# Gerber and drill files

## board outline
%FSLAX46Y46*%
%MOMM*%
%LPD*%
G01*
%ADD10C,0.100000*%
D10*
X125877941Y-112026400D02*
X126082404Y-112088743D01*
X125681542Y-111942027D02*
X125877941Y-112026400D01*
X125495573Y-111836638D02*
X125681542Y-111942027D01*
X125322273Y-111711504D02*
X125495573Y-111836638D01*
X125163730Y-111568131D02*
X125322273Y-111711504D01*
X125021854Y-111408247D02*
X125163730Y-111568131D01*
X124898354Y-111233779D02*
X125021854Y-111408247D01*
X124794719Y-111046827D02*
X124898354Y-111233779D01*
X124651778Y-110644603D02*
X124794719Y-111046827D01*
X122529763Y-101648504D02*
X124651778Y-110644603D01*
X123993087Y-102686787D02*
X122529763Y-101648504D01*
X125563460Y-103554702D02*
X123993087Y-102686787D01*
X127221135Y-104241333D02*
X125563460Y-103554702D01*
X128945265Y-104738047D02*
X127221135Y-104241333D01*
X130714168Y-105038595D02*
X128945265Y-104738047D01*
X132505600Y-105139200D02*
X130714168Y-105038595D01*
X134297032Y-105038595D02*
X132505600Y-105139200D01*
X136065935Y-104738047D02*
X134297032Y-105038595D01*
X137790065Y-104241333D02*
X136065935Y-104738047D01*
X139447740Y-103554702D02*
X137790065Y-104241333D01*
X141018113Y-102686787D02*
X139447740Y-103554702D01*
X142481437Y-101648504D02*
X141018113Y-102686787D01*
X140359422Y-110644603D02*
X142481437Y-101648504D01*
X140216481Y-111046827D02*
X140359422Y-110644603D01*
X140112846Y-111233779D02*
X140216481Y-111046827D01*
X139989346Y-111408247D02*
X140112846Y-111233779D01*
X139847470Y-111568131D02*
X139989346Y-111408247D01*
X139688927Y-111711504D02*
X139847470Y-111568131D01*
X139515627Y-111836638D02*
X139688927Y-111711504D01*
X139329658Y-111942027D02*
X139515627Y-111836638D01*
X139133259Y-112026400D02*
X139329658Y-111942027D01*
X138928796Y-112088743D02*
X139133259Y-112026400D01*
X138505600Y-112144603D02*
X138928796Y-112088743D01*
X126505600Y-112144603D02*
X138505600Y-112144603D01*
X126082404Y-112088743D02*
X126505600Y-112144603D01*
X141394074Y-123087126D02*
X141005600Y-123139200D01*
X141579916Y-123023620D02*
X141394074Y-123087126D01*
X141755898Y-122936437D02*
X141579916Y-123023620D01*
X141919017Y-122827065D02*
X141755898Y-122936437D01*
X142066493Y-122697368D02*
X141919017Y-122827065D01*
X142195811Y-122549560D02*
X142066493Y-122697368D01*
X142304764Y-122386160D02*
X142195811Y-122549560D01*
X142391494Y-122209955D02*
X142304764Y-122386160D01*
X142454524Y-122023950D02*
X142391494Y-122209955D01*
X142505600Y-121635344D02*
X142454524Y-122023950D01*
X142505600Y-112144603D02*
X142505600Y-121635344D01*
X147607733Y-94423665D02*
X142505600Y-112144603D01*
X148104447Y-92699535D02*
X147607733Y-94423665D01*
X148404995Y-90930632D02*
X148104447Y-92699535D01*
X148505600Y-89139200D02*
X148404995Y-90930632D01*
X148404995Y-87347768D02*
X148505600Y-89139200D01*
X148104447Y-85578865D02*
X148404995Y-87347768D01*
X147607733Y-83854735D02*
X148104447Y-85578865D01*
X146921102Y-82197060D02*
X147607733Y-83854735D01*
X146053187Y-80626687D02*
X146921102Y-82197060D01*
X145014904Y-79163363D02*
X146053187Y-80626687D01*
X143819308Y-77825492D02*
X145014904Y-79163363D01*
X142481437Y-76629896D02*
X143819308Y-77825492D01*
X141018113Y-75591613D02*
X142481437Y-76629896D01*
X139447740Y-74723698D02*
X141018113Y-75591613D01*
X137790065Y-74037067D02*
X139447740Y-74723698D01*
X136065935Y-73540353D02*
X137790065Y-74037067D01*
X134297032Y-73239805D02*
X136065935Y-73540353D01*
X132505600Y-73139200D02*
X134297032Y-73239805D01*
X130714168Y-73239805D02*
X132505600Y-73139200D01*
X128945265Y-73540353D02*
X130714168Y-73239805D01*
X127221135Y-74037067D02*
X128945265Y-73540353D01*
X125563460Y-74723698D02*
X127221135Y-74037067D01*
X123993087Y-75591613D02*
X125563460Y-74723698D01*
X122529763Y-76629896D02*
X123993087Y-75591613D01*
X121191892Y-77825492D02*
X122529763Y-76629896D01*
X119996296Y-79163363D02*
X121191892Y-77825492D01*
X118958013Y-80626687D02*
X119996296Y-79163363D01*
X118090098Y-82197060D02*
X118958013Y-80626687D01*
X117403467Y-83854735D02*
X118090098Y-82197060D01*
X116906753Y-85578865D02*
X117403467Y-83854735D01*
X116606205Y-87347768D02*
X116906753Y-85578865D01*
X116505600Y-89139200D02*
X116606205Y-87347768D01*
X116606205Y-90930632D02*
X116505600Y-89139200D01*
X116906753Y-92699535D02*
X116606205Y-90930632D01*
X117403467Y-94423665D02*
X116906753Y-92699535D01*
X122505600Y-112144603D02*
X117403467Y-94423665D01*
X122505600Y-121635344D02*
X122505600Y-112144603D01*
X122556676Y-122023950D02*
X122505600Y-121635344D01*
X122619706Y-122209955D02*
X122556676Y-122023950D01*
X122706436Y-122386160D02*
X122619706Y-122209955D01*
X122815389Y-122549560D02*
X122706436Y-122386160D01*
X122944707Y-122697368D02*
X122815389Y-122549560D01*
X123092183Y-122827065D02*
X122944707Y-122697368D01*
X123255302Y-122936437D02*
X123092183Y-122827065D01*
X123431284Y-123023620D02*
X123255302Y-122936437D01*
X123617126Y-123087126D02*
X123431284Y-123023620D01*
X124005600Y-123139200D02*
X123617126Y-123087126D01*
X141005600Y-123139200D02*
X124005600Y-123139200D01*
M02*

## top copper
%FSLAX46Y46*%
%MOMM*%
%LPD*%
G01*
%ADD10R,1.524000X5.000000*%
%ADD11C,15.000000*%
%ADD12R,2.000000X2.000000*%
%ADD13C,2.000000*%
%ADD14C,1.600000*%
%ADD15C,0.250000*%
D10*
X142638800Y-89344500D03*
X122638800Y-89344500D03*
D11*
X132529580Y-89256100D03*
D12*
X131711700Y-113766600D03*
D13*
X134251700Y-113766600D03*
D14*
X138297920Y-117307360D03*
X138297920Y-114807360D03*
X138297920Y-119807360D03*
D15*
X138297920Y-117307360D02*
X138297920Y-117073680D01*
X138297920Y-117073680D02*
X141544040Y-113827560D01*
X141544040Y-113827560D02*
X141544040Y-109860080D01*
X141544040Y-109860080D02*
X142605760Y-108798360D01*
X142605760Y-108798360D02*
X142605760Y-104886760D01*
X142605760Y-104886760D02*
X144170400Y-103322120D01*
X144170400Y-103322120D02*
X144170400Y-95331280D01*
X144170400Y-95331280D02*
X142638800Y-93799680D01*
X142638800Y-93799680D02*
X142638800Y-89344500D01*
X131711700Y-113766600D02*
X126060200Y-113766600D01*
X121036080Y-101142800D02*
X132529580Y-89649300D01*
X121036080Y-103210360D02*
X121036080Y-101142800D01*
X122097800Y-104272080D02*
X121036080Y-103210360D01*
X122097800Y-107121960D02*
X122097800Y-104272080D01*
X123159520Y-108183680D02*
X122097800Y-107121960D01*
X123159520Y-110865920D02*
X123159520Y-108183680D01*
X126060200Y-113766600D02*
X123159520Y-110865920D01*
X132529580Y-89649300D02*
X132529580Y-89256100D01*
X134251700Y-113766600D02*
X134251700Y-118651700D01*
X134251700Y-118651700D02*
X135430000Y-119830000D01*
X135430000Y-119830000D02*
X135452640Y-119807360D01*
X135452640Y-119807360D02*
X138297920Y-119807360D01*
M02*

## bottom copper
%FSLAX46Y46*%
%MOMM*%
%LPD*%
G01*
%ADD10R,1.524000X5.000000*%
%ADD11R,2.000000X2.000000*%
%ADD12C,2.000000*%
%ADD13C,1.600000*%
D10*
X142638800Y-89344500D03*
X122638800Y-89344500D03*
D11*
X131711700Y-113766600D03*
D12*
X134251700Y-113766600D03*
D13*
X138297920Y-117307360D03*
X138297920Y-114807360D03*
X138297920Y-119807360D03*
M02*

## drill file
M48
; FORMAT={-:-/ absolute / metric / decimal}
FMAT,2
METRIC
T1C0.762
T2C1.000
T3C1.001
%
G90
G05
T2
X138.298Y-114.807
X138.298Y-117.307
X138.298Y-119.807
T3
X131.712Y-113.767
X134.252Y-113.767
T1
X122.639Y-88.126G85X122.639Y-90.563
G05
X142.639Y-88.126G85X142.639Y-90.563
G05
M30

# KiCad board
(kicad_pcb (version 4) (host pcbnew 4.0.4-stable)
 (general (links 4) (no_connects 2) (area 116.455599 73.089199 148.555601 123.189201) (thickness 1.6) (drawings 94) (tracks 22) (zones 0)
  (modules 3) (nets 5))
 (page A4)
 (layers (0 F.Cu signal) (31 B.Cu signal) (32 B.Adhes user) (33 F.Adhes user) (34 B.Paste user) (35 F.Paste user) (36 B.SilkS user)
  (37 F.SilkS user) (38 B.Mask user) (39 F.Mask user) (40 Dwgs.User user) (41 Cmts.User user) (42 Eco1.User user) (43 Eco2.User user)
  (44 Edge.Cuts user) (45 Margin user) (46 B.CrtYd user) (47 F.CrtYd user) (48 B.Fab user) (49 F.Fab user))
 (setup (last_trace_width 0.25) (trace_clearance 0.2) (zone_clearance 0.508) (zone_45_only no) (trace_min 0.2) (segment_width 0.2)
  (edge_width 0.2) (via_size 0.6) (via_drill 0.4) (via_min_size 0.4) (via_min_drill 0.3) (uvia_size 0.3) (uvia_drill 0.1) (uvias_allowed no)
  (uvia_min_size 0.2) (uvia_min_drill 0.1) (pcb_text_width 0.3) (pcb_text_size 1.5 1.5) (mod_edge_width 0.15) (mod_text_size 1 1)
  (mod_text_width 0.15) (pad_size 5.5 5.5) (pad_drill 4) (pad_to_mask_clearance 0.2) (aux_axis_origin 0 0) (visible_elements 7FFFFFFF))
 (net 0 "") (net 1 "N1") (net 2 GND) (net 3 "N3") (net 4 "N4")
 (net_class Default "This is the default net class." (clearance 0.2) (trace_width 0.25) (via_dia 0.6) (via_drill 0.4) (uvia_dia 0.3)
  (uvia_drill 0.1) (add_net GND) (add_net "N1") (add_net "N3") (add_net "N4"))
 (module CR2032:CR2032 (layer F.Cu) (at 132.6388 89.3445)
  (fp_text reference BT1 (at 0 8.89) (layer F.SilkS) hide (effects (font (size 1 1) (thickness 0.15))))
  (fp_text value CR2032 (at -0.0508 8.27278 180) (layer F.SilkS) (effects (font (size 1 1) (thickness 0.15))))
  (pad 1 thru_hole rect (at 10 0) (size 1.524 5) (drill oval 0.762 3.2) (layers *.Cu *.Mask F.SilkS) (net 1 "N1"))
  (pad 1 thru_hole rect (at -10 0) (size 1.524 5) (drill oval 0.762 3.2) (layers *.Cu *.Mask F.SilkS) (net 1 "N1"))
  (pad 2 smd circle (at -0.10922 -0.0884) (size 15 15) (layers F.Cu F.Paste F.Mask) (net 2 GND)))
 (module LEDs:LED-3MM (layer F.Cu) (at 131.7117 113.7666)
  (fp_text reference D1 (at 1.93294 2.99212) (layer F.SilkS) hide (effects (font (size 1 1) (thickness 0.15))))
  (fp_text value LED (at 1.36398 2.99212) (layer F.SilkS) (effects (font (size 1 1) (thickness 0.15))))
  (pad 1 thru_hole rect (at 0 0 90) (size 2 2) (drill 1.00076) (layers *.Cu *.Mask F.SilkS) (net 2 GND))
  (pad 2 thru_hole circle (at 2.54 0) (size 2 2) (drill 1.00076) (layers *.Cu *.Mask F.SilkS) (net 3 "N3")))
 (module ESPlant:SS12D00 (layer F.Cu) (at 138.29792 117.30736 270)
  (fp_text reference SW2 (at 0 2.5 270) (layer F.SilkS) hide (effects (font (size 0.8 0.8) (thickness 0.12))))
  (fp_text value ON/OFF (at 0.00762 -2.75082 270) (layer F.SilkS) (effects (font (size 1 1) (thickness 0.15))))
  (pad 2 thru_hole circle (at 0 0 270) (size 1.6 1.6) (drill 1) (layers *.Cu *.Mask F.SilkS) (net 1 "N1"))
  (pad 1 thru_hole circle (at -2.5 0 270) (size 1.6 1.6) (drill 1) (layers *.Cu *.Mask F.SilkS) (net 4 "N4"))
  (pad 3 thru_hole circle (at 2.5 0 270) (size 1.6 1.6) (drill 1) (layers *.Cu *.Mask F.SilkS) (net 3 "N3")))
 (gr_line (start 125.877941 112.0264) (end 126.082404 112.088743) (layer Edge.Cuts) (width 0.1))
 (gr_line (start 125.681542 111.942027) (end 125.877941 112.0264) (layer Edge.Cuts) (width 0.1))
 (gr_line (start 125.495573 111.836638) (end 125.681542 111.942027) (layer Edge.Cuts) (width 0.1))
 (gr_line (start 125.322273 111.711504) (end 125.495573 111.836638) (layer Edge.Cuts) (width 0.1))
 (gr_line (start 125.16373 111.568131) (end 125.322273 111.711504) (layer Edge.Cuts) (width 0.1))
 (gr_line (start 125.021854 111.408247) (end 125.16373 111.568131) (layer Edge.Cuts) (width 0.1))
 (gr_line (start 124.898354 111.233779) (end 125.021854 111.408247) (layer Edge.Cuts) (width 0.1))
 (gr_line (start 124.794719 111.046827) (end 124.898354 111.233779) (layer Edge.Cuts) (width 0.1))
 (gr_line (start 124.651778 110.644603) (end 124.794719 111.046827) (layer Edge.Cuts) (width 0.1))
 (gr_line (start 122.529763 101.648504) (end 124.651778 110.644603) (layer Edge.Cuts) (width 0.1))
 (gr_line (start 123.993087 102.686787) (end 122.529763 101.648504) (layer Edge.Cuts) (width 0.1))
 (gr_line (start 125.56346 103.554702) (end 123.993087 102.686787) (layer Edge.Cuts) (width 0.1))
 (gr_line (start 127.221135 104.241333) (end 125.56346 103.554702) (layer Edge.Cuts) (width 0.1))
 (gr_line (start 128.945265 104.738047) (end 127.221135 104.241333) (layer Edge.Cuts) (width 0.1))
 (gr_line (start 130.714168 105.038595) (end 128.945265 104.738047) (layer Edge.Cuts) (width 0.1))
 (gr_line (start 132.5056 105.1392) (end 130.714168 105.038595) (layer Edge.Cuts) (width 0.1))
 (gr_line (start 134.297032 105.038595) (end 132.5056 105.1392) (layer Edge.Cuts) (width 0.1))
 (gr_line (start 136.065935 104.738047) (end 134.297032 105.038595) (layer Edge.Cuts) (width 0.1))
 (gr_line (start 137.790065 104.241333) (end 136.065935 104.738047) (layer Edge.Cuts) (width 0.1))
 (gr_line (start 139.44774 103.554702) (end 137.790065 104.241333) (layer Edge.Cuts) (width 0.1))
 (gr_line (start 141.018113 102.686787) (end 139.44774 103.554702) (layer Edge.Cuts) (width 0.1))
 (gr_line (start 142.481437 101.648504) (end 141.018113 102.686787) (layer Edge.Cuts) (width 0.1))
 (gr_line (start 140.359422 110.644603) (end 142.481437 101.648504) (layer Edge.Cuts) (width 0.1))
 (gr_line (start 140.216481 111.046827) (end 140.359422 110.644603) (layer Edge.Cuts) (width 0.1))
 (gr_line (start 140.112846 111.233779) (end 140.216481 111.046827) (layer Edge.Cuts) (width 0.1))
 (gr_line (start 139.989346 111.408247) (end 140.112846 111.233779) (layer Edge.Cuts) (width 0.1))
 (gr_line (start 139.84747 111.568131) (end 139.989346 111.408247) (layer Edge.Cuts) (width 0.1))
 (gr_line (start 139.688927 111.711504) (end 139.84747 111.568131) (layer Edge.Cuts) (width 0.1))
 (gr_line (start 139.515627 111.836638) (end 139.688927 111.711504) (layer Edge.Cuts) (width 0.1))
 (gr_line (start 139.329658 111.942027) (end 139.515627 111.836638) (layer Edge.Cuts) (width 0.1))
 (gr_line (start 139.133259 112.0264) (end 139.329658 111.942027) (layer Edge.Cuts) (width 0.1))
 (gr_line (start 138.928796 112.088743) (end 139.133259 112.0264) (layer Edge.Cuts) (width 0.1))
 (gr_line (start 138.5056 112.144603) (end 138.928796 112.088743) (layer Edge.Cuts) (width 0.1))
 (gr_line (start 126.5056 112.144603) (end 138.5056 112.144603) (layer Edge.Cuts) (width 0.1))
 (gr_line (start 126.082404 112.088743) (end 126.5056 112.144603) (layer Edge.Cuts) (width 0.1))
 (gr_line (start 141.394074 123.087126) (end 141.0056 123.1392) (layer Edge.Cuts) (width 0.1))
 (gr_line (start 141.579916 123.02362) (end 141.394074 123.087126) (layer Edge.Cuts) (width 0.1))
 (gr_line (start 141.755898 122.936437) (end 141.579916 123.02362) (layer Edge.Cuts) (width 0.1))
 (gr_line (start 141.919017 122.827065) (end 141.755898 122.936437) (layer Edge.Cuts) (width 0.1))
 (gr_line (start 142.066493 122.697368) (end 141.919017 122.827065) (layer Edge.Cuts) (width 0.1))
 (gr_line (start 142.195811 122.54956) (end 142.066493 122.697368) (layer Edge.Cuts) (width 0.1))
 (gr_line (start 142.304764 122.38616) (end 142.195811 122.54956) (layer Edge.Cuts) (width 0.1))
 (gr_line (start 142.391494 122.209955) (end 142.304764 122.38616) (layer Edge.Cuts) (width 0.1))
 (gr_line (start 142.454524 122.02395) (end 142.391494 122.209955) (layer Edge.Cuts) (width 0.1))
 (gr_line (start 142.5056 121.635344) (end 142.454524 122.02395) (layer Edge.Cuts) (width 0.1))
 (gr_line (start 142.5056 112.144603) (end 142.5056 121.635344) (layer Edge.Cuts) (width 0.1))
 (gr_line (start 147.607733 94.423665) (end 142.5056 112.144603) (layer Edge.Cuts) (width 0.1))
 (gr_line (start 148.104447 92.699535) (end 147.607733 94.423665) (layer Edge.Cuts) (width 0.1))
 (gr_line (start 148.404995 90.930632) (end 148.104447 92.699535) (layer Edge.Cuts) (width 0.1))
 (gr_line (start 148.5056 89.1392) (end 148.404995 90.930632) (layer Edge.Cuts) (width 0.1))
 (gr_line (start 148.404995 87.347768) (end 148.5056 89.1392) (layer Edge.Cuts) (width 0.1))
 (gr_line (start 148.104447 85.578865) (end 148.404995 87.347768) (layer Edge.Cuts) (width 0.1))
 (gr_line (start 147.607733 83.854735) (end 148.104447 85.578865) (layer Edge.Cuts) (width 0.1))
 (gr_line (start 146.921102 82.19706) (end 147.607733 83.854735) (layer Edge.Cuts) (width 0.1))
 (gr_line (start 146.053187 80.626687) (end 146.921102 82.19706) (layer Edge.Cuts) (width 0.1))
 (gr_line (start 145.014904 79.163363) (end 146.053187 80.626687) (layer Edge.Cuts) (width 0.1))
 (gr_line (start 143.819308 77.825492) (end 145.014904 79.163363) (layer Edge.Cuts) (width 0.1))
 (gr_line (start 142.481437 76.629896) (end 143.819308 77.825492) (layer Edge.Cuts) (width 0.1))
 (gr_line (start 141.018113 75.591613) (end 142.481437 76.629896) (layer Edge.Cuts) (width 0.1))
 (gr_line (start 139.44774 74.723698) (end 141.018113 75.591613) (layer Edge.Cuts) (width 0.1))
 (gr_line (start 137.790065 74.037067) (end 139.44774 74.723698) (layer Edge.Cuts) (width 0.1))
 (gr_line (start 136.065935 73.540353) (end 137.790065 74.037067) (layer Edge.Cuts) (width 0.1))
 (gr_line (start 134.297032 73.239805) (end 136.065935 73.540353) (layer Edge.Cuts) (width 0.1))
 (gr_line (start 132.5056 73.1392) (end 134.297032 73.239805) (layer Edge.Cuts) (width 0.1))
 (gr_line (start 130.714168 73.239805) (end 132.5056 73.1392) (layer Edge.Cuts) (width 0.1))
 (gr_line (start 128.945265 73.540353) (end 130.714168 73.239805) (layer Edge.Cuts) (width 0.1))
 (gr_line (start 127.221135 74.037067) (end 128.945265 73.540353) (layer Edge.Cuts) (width 0.1))
 (gr_line (start 125.56346 74.723698) (end 127.221135 74.037067) (layer Edge.Cuts) (width 0.1))
 (gr_line (start 123.993087 75.591613) (end 125.56346 74.723698) (layer Edge.Cuts) (width 0.1))
 (gr_line (start 122.529763 76.629896) (end 123.993087 75.591613) (layer Edge.Cuts) (width 0.1))
 (gr_line (start 121.191892 77.825492) (end 122.529763 76.629896) (layer Edge.Cuts) (width 0.1))
 (gr_line (start 119.996296 79.163363) (end 121.191892 77.825492) (layer Edge.Cuts) (width 0.1))
 (gr_line (start 118.958013 80.626687) (end 119.996296 79.163363) (layer Edge.Cuts) (width 0.1))
 (gr_line (start 118.090098 82.19706) (end 118.958013 80.626687) (layer Edge.Cuts) (width 0.1))
 (gr_line (start 117.403467 83.854735) (end 118.090098 82.19706) (layer Edge.Cuts) (width 0.1))
 (gr_line (start 116.906753 85.578865) (end 117.403467 83.854735) (layer Edge.Cuts) (width 0.1))
 (gr_line (start 116.606205 87.347768) (end 116.906753 85.578865) (layer Edge.Cuts) (width 0.1))
 (gr_line (start 116.5056 89.1392) (end 116.606205 87.347768) (layer Edge.Cuts) (width 0.1))
 (gr_line (start 116.606205 90.930632) (end 116.5056 89.1392) (layer Edge.Cuts) (width 0.1))
 (gr_line (start 116.906753 92.699535) (end 116.606205 90.930632) (layer Edge.Cuts) (width 0.1))
 (gr_line (start 117.403467 94.423665) (end 116.906753 92.699535) (layer Edge.Cuts) (width 0.1))
 (gr_line (start 122.5056 112.144603) (end 117.403467 94.423665) (layer Edge.Cuts) (width 0.1))
 (gr_line (start 122.5056 121.635344) (end 122.5056 112.144603) (layer Edge.Cuts) (width 0.1))
 (gr_line (start 122.556676 122.02395) (end 122.5056 121.635344) (layer Edge.Cuts) (width 0.1))
 (gr_line (start 122.619706 122.209955) (end 122.556676 122.02395) (layer Edge.Cuts) (width 0.1))
 (gr_line (start 122.706436 122.38616) (end 122.619706 122.209955) (layer Edge.Cuts) (width 0.1))
 (gr_line (start 122.815389 122.54956) (end 122.706436 122.38616) (layer Edge.Cuts) (width 0.1))
 (gr_line (start 122.944707 122.697368) (end 122.815389 122.54956) (layer Edge.Cuts) (width 0.1))
 (gr_line (start 123.092183 122.827065) (end 122.944707 122.697368) (layer Edge.Cuts) (width 0.1))
 (gr_line (start 123.255302 122.936437) (end 123.092183 122.827065) (layer Edge.Cuts) (width 0.1))
 (gr_line (start 123.431284 123.02362) (end 123.255302 122.936437) (layer Edge.Cuts) (width 0.1))
 (gr_line (start 123.617126 123.087126) (end 123.431284 123.02362) (layer Edge.Cuts) (width 0.1))
 (gr_line (start 124.0056 123.1392) (end 123.617126 123.087126) (layer Edge.Cuts) (width 0.1))
 (gr_line (start 141.0056 123.1392) (end 124.0056 123.1392) (layer Edge.Cuts) (width 0.1))
 (segment (start 138.29792 117.30736) (end 138.29792 117.07368) (width 0.25) (layer F.Cu) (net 1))
 (segment (start 138.29792 117.07368) (end 141.54404 113.82756) (width 0.25) (layer F.Cu) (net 1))
 (segment (start 141.54404 113.82756) (end 141.54404 109.86008) (width 0.25) (layer F.Cu) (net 1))
 (segment (start 141.54404 109.86008) (end 142.60576 108.79836) (width 0.25) (layer F.Cu) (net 1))
 (segment (start 142.60576 108.79836) (end 142.60576 104.88676) (width 0.25) (layer F.Cu) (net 1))
 (segment (start 142.60576 104.88676) (end 144.1704 103.32212) (width 0.25) (layer F.Cu) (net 1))
 (segment (start 144.1704 103.32212) (end 144.1704 95.33128) (width 0.25) (layer F.Cu) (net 1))
 (segment (start 144.1704 95.33128) (end 142.6388 93.79968) (width 0.25) (layer F.Cu) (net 1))
 (segment (start 142.6388 93.79968) (end 142.6388 89.3445) (width 0.25) (layer F.Cu) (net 1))
 (segment (start 131.7117 113.7666) (end 126.0602 113.7666) (width 0.25) (layer F.Cu) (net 2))
 (segment (start 121.03608 101.1428) (end 132.52958 89.6493) (width 0.25) (layer F.Cu) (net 2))
 (segment (start 121.03608 103.21036) (end 121.03608 101.1428) (width 0.25) (layer F.Cu) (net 2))
 (segment (start 122.0978 104.27208) (end 121.03608 103.21036) (width 0.25) (layer F.Cu) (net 2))
 (segment (start 122.0978 107.12196) (end 122.0978 104.27208) (width 0.25) (layer F.Cu) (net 2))
 (segment (start 123.15952 108.18368) (end 122.0978 107.12196) (width 0.25) (layer F.Cu) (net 2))
 (segment (start 123.15952 110.86592) (end 123.15952 108.18368) (width 0.25) (layer F.Cu) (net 2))
 (segment (start 126.0602 113.7666) (end 123.15952 110.86592) (width 0.25) (layer F.Cu) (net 2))
 (segment (start 132.52958 89.6493) (end 132.52958 89.2561) (width 0.25) (layer F.Cu) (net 2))
 (segment (start 134.2517 113.7666) (end 134.2517 118.6517) (width 0.25) (layer F.Cu) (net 3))
 (segment (start 134.2517 118.6517) (end 135.43 119.83) (width 0.25) (layer F.Cu) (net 3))
 (segment (start 135.43 119.83) (end 135.45264 119.80736) (width 0.25) (layer F.Cu) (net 3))
 (segment (start 135.45264 119.80736) (end 138.29792 119.80736) (width 0.25) (layer F.Cu) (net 3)))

